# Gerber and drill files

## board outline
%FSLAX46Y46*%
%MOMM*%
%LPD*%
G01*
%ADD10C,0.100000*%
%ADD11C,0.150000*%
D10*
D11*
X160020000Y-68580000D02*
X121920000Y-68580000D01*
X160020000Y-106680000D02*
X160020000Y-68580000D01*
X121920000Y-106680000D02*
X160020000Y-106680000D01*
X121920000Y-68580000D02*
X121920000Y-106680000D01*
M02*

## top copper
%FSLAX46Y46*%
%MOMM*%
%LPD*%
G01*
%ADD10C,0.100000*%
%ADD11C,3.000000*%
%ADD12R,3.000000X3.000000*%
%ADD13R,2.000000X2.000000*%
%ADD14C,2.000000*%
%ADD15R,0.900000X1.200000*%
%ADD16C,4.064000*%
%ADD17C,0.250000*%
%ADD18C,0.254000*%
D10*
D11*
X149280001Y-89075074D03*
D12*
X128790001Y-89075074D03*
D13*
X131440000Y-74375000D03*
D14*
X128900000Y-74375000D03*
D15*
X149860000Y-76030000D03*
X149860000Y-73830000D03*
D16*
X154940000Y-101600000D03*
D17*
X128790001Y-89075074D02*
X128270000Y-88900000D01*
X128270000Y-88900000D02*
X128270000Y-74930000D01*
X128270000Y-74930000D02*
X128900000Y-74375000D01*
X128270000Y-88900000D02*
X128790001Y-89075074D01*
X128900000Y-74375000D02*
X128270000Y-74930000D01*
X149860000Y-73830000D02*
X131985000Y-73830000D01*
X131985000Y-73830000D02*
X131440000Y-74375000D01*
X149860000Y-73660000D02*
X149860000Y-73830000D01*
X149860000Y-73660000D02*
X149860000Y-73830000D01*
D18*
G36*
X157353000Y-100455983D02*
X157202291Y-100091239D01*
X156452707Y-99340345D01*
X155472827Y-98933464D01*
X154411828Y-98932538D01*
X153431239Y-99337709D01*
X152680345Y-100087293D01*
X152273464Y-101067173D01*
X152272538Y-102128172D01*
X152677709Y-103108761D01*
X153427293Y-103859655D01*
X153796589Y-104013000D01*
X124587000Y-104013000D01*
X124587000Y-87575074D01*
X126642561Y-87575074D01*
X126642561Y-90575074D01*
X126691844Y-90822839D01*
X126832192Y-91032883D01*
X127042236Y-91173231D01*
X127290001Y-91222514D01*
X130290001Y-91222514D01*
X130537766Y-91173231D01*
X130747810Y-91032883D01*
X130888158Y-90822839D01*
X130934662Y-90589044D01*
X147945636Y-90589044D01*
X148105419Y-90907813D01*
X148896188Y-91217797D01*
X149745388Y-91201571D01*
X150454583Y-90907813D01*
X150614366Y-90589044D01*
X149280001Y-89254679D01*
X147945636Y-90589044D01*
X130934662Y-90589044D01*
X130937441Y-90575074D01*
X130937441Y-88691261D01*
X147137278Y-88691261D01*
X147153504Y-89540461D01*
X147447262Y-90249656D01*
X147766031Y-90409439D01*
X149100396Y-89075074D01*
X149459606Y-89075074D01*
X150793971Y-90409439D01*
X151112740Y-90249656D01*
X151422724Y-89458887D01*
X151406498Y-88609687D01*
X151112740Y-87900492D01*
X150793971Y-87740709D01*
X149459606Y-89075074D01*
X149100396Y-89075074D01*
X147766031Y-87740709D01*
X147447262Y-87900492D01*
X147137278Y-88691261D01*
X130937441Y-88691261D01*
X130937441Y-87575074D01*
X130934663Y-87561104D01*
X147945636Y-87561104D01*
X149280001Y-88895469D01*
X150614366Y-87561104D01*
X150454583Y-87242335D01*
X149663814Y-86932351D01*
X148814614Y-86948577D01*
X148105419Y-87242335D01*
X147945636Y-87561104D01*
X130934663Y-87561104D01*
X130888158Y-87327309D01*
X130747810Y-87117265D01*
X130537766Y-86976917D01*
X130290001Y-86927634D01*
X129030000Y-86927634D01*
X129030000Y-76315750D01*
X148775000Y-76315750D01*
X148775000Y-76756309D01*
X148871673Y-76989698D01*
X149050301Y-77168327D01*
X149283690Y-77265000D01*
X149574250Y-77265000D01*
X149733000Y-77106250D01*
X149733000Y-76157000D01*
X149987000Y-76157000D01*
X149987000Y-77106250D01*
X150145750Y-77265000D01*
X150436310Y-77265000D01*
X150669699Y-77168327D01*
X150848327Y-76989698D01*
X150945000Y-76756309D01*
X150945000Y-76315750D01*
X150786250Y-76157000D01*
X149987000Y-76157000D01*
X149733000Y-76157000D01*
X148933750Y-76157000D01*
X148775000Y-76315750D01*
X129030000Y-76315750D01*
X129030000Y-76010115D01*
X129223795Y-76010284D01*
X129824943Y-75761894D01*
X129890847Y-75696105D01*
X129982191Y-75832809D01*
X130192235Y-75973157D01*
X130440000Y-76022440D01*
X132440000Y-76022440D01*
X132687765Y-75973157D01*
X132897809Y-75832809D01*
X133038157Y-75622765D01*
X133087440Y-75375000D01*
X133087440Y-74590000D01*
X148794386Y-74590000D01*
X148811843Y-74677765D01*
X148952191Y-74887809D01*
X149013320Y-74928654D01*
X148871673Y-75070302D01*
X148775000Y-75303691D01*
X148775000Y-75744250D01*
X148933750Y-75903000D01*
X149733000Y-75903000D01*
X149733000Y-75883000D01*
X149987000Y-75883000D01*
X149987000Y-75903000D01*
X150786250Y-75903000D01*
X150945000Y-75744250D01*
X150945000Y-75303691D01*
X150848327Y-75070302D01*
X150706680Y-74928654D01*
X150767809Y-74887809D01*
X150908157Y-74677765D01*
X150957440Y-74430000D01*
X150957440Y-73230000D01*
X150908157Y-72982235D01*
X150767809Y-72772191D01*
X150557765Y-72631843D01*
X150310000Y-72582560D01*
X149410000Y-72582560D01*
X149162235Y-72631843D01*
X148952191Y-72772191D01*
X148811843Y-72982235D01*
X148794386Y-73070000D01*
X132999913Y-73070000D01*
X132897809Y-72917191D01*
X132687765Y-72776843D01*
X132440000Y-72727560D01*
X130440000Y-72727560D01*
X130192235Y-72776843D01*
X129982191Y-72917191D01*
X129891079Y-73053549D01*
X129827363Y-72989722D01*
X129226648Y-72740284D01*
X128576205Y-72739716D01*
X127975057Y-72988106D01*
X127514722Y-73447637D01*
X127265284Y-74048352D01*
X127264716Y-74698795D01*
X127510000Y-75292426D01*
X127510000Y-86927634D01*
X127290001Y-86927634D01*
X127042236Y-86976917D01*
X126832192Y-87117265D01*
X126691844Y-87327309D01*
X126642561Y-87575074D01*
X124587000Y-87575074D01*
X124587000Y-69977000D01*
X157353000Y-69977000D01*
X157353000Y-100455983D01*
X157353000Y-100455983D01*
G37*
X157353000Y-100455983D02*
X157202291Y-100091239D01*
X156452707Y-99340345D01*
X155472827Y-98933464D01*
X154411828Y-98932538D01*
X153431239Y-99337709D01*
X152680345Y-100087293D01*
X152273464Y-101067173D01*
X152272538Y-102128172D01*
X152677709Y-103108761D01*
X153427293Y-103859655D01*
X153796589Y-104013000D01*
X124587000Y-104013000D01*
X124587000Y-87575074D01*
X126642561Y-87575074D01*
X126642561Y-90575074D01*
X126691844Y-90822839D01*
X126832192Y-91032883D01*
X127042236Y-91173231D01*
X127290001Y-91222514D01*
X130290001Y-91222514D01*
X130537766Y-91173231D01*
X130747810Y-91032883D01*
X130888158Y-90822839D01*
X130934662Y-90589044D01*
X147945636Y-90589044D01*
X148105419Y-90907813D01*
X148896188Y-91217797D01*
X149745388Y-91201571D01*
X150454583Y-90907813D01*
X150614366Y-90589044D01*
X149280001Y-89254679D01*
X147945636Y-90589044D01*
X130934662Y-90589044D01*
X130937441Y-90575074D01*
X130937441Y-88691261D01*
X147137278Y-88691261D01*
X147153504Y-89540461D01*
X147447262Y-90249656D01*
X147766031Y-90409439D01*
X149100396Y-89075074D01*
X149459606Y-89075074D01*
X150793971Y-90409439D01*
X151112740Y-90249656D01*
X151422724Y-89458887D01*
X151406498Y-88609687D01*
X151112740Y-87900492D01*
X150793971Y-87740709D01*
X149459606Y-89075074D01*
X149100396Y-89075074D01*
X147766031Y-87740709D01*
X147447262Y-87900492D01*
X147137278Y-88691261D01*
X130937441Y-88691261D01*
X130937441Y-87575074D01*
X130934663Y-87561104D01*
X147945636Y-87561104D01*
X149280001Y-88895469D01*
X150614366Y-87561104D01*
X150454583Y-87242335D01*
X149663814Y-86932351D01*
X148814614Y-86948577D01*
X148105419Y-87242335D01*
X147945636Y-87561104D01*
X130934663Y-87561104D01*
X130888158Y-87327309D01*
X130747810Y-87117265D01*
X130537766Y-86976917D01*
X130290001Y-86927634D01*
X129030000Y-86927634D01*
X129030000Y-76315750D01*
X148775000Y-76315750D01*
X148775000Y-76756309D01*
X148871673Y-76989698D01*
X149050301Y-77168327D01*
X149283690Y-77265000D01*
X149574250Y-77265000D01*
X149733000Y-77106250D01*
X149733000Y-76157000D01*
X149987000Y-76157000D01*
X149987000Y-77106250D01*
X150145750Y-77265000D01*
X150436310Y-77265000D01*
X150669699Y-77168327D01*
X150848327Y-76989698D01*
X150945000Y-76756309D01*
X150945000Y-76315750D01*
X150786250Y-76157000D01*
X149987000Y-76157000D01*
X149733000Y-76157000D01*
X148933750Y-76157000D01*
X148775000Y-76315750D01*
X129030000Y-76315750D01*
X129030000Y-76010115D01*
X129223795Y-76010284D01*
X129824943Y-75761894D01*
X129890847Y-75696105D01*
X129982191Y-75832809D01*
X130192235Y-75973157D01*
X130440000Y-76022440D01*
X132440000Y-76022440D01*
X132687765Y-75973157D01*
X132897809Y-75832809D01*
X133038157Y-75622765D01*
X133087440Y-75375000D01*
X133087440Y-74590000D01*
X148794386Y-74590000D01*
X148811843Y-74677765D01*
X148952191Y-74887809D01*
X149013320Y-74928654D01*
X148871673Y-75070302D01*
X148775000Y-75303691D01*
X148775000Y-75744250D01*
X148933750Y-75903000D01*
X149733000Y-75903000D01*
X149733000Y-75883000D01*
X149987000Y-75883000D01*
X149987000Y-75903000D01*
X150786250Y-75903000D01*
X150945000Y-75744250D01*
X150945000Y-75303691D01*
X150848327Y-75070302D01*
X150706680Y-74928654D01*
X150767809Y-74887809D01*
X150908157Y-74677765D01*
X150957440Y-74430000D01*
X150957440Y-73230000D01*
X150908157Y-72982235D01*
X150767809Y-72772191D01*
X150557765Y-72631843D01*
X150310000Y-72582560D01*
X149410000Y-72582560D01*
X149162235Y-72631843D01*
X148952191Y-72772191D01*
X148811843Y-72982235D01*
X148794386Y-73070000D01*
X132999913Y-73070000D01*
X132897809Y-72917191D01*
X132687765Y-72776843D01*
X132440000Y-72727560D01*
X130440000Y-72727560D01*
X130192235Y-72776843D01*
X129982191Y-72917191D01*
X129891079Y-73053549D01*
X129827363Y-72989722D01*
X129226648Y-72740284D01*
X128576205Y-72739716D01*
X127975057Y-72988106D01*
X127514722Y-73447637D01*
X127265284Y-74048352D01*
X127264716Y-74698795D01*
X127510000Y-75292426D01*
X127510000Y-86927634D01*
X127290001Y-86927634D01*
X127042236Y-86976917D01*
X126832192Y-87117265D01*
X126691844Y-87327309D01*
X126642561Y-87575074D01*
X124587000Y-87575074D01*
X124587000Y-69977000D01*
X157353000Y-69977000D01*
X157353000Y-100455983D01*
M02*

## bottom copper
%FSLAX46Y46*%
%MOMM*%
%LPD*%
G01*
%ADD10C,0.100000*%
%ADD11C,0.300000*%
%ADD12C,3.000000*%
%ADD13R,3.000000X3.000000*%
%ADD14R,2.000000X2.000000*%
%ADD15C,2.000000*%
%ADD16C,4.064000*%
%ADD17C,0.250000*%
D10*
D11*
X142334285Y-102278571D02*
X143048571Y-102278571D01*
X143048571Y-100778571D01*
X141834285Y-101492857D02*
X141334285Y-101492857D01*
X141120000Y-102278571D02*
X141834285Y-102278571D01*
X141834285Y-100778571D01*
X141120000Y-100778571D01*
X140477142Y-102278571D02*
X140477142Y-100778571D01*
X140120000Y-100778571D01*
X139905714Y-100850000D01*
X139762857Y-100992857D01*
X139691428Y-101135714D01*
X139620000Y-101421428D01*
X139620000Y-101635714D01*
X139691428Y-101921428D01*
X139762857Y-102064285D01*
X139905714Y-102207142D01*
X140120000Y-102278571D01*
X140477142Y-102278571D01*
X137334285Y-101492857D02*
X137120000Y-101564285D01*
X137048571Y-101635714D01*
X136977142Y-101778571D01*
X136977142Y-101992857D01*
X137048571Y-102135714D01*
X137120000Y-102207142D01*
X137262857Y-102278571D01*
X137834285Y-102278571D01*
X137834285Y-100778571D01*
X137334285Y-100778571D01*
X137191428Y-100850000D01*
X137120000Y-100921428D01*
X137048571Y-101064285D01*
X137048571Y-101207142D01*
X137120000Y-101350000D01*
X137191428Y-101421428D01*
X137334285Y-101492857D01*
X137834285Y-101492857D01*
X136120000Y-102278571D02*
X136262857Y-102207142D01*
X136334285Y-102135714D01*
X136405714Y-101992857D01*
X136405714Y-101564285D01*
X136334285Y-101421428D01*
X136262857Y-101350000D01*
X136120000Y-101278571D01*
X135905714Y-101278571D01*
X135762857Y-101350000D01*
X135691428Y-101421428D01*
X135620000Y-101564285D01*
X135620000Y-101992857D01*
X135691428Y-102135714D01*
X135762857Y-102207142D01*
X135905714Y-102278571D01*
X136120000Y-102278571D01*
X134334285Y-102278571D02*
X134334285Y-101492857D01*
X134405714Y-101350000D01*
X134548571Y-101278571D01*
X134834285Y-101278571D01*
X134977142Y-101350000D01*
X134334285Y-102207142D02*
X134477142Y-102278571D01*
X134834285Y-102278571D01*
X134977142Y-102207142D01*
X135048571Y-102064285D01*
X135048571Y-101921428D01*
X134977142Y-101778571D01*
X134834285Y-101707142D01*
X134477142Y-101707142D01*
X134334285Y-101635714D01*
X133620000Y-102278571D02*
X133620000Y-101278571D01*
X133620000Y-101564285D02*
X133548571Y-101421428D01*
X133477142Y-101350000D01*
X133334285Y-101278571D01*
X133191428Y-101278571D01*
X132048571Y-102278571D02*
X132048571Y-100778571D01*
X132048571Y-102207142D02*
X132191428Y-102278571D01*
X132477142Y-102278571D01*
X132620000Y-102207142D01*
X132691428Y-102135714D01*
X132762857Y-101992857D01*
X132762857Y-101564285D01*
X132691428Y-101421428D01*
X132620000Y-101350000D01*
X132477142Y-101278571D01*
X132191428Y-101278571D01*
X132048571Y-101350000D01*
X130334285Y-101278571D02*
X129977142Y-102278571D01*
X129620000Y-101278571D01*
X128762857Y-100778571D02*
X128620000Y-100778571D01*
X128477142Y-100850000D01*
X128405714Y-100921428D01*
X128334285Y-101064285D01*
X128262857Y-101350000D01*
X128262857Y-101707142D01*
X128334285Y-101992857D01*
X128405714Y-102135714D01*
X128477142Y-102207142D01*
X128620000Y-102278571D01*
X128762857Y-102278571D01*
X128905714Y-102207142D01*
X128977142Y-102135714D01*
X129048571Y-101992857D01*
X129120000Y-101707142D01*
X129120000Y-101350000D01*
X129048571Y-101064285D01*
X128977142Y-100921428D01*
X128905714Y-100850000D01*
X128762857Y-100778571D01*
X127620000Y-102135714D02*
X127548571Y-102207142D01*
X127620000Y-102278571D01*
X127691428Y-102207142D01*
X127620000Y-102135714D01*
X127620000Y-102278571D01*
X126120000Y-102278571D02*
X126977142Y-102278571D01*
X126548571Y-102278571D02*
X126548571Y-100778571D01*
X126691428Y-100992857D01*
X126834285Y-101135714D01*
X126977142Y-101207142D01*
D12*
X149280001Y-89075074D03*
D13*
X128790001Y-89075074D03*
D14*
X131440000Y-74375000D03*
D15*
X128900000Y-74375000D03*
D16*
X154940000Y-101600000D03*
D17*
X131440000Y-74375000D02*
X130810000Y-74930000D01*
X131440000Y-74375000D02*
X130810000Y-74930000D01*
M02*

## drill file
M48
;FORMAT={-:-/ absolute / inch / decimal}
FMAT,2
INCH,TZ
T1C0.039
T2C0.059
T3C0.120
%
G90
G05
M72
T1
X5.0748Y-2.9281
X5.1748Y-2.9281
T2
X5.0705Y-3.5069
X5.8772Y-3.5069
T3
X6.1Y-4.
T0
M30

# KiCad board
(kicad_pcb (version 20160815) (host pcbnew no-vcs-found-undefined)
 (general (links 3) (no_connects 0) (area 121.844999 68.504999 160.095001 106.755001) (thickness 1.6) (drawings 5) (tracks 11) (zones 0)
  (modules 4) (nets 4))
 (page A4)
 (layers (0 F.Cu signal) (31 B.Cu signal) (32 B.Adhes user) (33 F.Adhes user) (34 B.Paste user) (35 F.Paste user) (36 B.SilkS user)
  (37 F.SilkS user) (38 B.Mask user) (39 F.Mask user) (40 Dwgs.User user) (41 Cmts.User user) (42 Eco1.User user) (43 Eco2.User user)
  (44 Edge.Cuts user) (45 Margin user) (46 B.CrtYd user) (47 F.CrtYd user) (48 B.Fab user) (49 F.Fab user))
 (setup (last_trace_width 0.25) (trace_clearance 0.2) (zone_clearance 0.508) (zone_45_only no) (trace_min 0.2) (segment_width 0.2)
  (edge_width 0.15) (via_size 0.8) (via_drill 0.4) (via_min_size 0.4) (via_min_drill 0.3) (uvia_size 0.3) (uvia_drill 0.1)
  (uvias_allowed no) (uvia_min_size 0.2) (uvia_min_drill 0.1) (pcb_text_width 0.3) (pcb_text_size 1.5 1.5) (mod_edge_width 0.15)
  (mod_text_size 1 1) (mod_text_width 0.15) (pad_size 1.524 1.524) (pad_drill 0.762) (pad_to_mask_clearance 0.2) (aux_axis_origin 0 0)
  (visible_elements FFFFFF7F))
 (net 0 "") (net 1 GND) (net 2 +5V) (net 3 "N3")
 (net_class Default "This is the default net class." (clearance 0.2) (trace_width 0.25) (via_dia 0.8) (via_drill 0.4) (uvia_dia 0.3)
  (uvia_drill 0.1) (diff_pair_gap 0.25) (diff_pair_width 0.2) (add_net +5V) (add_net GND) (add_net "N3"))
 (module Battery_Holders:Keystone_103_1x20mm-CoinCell (layer F.Cu) (at 128.790001 89.075074)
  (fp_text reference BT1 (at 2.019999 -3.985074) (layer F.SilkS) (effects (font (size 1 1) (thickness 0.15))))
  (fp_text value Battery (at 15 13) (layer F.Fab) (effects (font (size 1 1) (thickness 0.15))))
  (pad 2 thru_hole circle (at 20.49 0) (size 3 3) (drill 1.5) (layers *.Cu *.Mask F.SilkS) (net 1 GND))
  (pad 1 thru_hole rect (at 0 0) (size 3 3) (drill 1.5) (layers *.Cu *.Mask F.SilkS) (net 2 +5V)))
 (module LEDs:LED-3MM (layer F.Cu) (at 131.44 74.375 180)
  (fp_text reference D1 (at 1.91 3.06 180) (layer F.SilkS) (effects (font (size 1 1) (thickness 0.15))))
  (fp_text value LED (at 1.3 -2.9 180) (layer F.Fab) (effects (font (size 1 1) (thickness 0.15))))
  (pad 1 thru_hole rect (at 0 0 270) (size 2 2) (drill 1.00076) (layers *.Cu *.Mask F.SilkS) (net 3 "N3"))
  (pad 2 thru_hole circle (at 2.54 0 180) (size 2 2) (drill 1.00076) (layers *.Cu *.Mask F.SilkS) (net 2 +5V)))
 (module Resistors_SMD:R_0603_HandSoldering (layer F.Cu) (at 149.86 74.93 90)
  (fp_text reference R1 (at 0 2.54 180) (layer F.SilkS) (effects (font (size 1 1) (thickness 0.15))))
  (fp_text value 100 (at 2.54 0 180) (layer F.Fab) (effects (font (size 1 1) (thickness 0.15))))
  (pad 1 smd rect (at -1.1 0 90) (size 1.2 0.9) (layers F.Cu F.Paste F.Mask) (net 1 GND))
  (pad 2 smd rect (at 1.1 0 90) (size 1.2 0.9) (layers F.Cu F.Paste F.Mask) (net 3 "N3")))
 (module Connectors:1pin (layer F.Cu) (at 154.94 101.6)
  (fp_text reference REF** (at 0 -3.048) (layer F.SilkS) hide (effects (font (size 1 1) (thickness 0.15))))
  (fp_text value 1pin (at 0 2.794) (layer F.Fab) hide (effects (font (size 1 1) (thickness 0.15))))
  (pad 1 thru_hole circle (at 0 0) (size 4.064 4.064) (drill 3.048) (layers *.Cu *.Mask F.SilkS)))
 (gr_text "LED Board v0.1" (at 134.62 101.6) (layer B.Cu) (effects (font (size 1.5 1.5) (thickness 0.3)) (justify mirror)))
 (gr_line (start 160.02 68.58) (end 121.92 68.58) (angle 90) (layer Edge.Cuts) (width 0.15))
 (gr_line (start 160.02 106.68) (end 160.02 68.58) (angle 90) (layer Edge.Cuts) (width 0.15))
 (gr_line (start 121.92 106.68) (end 160.02 106.68) (angle 90) (layer Edge.Cuts) (width 0.15))
 (gr_line (start 121.92 68.58) (end 121.92 106.68) (angle 90) (layer Edge.Cuts) (width 0.15))
 (segment (start 128.790001 89.075074) (end 128.27 88.9) (width 0.25) (layer F.Cu) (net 2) (status 80000))
 (segment (start 128.27 88.9) (end 128.27 74.93) (width 0.25) (layer F.Cu) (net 2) (status 80000))
 (segment (start 128.27 74.93) (end 128.9 74.375) (width 0.25) (layer F.Cu) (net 2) (status 80000))
 (segment (start 128.27 88.9) (end 128.790001 89.075074) (width 0.25) (layer F.Cu) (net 2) (status 80000))
 (segment (start 128.9 74.375) (end 128.27 74.93) (width 0.25) (layer F.Cu) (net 2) (status 80000))
 (segment (start 149.86 73.83) (end 131.985 73.83) (width 0.25) (layer F.Cu) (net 3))
 (segment (start 131.985 73.83) (end 131.44 74.375) (width 0.25) (layer F.Cu) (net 3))
 (segment (start 149.86 73.66) (end 149.86 73.83) (width 0.25) (layer F.Cu) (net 3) (status 80000))
 (segment (start 149.86 73.66) (end 149.86 73.83) (width 0.25) (layer F.Cu) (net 3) (status 80000))
 (segment (start 131.44 74.375) (end 130.81 74.93) (width 0.25) (layer B.Cu) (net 3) (status 80000))
 (segment (start 131.44 74.375) (end 130.81 74.93) (width 0.25) (layer B.Cu) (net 3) (status 80000))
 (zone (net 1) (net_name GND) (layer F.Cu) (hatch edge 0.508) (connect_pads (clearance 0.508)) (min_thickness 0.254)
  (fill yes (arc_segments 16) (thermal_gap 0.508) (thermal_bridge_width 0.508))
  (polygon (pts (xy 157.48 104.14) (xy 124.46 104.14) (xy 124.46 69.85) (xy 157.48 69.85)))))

